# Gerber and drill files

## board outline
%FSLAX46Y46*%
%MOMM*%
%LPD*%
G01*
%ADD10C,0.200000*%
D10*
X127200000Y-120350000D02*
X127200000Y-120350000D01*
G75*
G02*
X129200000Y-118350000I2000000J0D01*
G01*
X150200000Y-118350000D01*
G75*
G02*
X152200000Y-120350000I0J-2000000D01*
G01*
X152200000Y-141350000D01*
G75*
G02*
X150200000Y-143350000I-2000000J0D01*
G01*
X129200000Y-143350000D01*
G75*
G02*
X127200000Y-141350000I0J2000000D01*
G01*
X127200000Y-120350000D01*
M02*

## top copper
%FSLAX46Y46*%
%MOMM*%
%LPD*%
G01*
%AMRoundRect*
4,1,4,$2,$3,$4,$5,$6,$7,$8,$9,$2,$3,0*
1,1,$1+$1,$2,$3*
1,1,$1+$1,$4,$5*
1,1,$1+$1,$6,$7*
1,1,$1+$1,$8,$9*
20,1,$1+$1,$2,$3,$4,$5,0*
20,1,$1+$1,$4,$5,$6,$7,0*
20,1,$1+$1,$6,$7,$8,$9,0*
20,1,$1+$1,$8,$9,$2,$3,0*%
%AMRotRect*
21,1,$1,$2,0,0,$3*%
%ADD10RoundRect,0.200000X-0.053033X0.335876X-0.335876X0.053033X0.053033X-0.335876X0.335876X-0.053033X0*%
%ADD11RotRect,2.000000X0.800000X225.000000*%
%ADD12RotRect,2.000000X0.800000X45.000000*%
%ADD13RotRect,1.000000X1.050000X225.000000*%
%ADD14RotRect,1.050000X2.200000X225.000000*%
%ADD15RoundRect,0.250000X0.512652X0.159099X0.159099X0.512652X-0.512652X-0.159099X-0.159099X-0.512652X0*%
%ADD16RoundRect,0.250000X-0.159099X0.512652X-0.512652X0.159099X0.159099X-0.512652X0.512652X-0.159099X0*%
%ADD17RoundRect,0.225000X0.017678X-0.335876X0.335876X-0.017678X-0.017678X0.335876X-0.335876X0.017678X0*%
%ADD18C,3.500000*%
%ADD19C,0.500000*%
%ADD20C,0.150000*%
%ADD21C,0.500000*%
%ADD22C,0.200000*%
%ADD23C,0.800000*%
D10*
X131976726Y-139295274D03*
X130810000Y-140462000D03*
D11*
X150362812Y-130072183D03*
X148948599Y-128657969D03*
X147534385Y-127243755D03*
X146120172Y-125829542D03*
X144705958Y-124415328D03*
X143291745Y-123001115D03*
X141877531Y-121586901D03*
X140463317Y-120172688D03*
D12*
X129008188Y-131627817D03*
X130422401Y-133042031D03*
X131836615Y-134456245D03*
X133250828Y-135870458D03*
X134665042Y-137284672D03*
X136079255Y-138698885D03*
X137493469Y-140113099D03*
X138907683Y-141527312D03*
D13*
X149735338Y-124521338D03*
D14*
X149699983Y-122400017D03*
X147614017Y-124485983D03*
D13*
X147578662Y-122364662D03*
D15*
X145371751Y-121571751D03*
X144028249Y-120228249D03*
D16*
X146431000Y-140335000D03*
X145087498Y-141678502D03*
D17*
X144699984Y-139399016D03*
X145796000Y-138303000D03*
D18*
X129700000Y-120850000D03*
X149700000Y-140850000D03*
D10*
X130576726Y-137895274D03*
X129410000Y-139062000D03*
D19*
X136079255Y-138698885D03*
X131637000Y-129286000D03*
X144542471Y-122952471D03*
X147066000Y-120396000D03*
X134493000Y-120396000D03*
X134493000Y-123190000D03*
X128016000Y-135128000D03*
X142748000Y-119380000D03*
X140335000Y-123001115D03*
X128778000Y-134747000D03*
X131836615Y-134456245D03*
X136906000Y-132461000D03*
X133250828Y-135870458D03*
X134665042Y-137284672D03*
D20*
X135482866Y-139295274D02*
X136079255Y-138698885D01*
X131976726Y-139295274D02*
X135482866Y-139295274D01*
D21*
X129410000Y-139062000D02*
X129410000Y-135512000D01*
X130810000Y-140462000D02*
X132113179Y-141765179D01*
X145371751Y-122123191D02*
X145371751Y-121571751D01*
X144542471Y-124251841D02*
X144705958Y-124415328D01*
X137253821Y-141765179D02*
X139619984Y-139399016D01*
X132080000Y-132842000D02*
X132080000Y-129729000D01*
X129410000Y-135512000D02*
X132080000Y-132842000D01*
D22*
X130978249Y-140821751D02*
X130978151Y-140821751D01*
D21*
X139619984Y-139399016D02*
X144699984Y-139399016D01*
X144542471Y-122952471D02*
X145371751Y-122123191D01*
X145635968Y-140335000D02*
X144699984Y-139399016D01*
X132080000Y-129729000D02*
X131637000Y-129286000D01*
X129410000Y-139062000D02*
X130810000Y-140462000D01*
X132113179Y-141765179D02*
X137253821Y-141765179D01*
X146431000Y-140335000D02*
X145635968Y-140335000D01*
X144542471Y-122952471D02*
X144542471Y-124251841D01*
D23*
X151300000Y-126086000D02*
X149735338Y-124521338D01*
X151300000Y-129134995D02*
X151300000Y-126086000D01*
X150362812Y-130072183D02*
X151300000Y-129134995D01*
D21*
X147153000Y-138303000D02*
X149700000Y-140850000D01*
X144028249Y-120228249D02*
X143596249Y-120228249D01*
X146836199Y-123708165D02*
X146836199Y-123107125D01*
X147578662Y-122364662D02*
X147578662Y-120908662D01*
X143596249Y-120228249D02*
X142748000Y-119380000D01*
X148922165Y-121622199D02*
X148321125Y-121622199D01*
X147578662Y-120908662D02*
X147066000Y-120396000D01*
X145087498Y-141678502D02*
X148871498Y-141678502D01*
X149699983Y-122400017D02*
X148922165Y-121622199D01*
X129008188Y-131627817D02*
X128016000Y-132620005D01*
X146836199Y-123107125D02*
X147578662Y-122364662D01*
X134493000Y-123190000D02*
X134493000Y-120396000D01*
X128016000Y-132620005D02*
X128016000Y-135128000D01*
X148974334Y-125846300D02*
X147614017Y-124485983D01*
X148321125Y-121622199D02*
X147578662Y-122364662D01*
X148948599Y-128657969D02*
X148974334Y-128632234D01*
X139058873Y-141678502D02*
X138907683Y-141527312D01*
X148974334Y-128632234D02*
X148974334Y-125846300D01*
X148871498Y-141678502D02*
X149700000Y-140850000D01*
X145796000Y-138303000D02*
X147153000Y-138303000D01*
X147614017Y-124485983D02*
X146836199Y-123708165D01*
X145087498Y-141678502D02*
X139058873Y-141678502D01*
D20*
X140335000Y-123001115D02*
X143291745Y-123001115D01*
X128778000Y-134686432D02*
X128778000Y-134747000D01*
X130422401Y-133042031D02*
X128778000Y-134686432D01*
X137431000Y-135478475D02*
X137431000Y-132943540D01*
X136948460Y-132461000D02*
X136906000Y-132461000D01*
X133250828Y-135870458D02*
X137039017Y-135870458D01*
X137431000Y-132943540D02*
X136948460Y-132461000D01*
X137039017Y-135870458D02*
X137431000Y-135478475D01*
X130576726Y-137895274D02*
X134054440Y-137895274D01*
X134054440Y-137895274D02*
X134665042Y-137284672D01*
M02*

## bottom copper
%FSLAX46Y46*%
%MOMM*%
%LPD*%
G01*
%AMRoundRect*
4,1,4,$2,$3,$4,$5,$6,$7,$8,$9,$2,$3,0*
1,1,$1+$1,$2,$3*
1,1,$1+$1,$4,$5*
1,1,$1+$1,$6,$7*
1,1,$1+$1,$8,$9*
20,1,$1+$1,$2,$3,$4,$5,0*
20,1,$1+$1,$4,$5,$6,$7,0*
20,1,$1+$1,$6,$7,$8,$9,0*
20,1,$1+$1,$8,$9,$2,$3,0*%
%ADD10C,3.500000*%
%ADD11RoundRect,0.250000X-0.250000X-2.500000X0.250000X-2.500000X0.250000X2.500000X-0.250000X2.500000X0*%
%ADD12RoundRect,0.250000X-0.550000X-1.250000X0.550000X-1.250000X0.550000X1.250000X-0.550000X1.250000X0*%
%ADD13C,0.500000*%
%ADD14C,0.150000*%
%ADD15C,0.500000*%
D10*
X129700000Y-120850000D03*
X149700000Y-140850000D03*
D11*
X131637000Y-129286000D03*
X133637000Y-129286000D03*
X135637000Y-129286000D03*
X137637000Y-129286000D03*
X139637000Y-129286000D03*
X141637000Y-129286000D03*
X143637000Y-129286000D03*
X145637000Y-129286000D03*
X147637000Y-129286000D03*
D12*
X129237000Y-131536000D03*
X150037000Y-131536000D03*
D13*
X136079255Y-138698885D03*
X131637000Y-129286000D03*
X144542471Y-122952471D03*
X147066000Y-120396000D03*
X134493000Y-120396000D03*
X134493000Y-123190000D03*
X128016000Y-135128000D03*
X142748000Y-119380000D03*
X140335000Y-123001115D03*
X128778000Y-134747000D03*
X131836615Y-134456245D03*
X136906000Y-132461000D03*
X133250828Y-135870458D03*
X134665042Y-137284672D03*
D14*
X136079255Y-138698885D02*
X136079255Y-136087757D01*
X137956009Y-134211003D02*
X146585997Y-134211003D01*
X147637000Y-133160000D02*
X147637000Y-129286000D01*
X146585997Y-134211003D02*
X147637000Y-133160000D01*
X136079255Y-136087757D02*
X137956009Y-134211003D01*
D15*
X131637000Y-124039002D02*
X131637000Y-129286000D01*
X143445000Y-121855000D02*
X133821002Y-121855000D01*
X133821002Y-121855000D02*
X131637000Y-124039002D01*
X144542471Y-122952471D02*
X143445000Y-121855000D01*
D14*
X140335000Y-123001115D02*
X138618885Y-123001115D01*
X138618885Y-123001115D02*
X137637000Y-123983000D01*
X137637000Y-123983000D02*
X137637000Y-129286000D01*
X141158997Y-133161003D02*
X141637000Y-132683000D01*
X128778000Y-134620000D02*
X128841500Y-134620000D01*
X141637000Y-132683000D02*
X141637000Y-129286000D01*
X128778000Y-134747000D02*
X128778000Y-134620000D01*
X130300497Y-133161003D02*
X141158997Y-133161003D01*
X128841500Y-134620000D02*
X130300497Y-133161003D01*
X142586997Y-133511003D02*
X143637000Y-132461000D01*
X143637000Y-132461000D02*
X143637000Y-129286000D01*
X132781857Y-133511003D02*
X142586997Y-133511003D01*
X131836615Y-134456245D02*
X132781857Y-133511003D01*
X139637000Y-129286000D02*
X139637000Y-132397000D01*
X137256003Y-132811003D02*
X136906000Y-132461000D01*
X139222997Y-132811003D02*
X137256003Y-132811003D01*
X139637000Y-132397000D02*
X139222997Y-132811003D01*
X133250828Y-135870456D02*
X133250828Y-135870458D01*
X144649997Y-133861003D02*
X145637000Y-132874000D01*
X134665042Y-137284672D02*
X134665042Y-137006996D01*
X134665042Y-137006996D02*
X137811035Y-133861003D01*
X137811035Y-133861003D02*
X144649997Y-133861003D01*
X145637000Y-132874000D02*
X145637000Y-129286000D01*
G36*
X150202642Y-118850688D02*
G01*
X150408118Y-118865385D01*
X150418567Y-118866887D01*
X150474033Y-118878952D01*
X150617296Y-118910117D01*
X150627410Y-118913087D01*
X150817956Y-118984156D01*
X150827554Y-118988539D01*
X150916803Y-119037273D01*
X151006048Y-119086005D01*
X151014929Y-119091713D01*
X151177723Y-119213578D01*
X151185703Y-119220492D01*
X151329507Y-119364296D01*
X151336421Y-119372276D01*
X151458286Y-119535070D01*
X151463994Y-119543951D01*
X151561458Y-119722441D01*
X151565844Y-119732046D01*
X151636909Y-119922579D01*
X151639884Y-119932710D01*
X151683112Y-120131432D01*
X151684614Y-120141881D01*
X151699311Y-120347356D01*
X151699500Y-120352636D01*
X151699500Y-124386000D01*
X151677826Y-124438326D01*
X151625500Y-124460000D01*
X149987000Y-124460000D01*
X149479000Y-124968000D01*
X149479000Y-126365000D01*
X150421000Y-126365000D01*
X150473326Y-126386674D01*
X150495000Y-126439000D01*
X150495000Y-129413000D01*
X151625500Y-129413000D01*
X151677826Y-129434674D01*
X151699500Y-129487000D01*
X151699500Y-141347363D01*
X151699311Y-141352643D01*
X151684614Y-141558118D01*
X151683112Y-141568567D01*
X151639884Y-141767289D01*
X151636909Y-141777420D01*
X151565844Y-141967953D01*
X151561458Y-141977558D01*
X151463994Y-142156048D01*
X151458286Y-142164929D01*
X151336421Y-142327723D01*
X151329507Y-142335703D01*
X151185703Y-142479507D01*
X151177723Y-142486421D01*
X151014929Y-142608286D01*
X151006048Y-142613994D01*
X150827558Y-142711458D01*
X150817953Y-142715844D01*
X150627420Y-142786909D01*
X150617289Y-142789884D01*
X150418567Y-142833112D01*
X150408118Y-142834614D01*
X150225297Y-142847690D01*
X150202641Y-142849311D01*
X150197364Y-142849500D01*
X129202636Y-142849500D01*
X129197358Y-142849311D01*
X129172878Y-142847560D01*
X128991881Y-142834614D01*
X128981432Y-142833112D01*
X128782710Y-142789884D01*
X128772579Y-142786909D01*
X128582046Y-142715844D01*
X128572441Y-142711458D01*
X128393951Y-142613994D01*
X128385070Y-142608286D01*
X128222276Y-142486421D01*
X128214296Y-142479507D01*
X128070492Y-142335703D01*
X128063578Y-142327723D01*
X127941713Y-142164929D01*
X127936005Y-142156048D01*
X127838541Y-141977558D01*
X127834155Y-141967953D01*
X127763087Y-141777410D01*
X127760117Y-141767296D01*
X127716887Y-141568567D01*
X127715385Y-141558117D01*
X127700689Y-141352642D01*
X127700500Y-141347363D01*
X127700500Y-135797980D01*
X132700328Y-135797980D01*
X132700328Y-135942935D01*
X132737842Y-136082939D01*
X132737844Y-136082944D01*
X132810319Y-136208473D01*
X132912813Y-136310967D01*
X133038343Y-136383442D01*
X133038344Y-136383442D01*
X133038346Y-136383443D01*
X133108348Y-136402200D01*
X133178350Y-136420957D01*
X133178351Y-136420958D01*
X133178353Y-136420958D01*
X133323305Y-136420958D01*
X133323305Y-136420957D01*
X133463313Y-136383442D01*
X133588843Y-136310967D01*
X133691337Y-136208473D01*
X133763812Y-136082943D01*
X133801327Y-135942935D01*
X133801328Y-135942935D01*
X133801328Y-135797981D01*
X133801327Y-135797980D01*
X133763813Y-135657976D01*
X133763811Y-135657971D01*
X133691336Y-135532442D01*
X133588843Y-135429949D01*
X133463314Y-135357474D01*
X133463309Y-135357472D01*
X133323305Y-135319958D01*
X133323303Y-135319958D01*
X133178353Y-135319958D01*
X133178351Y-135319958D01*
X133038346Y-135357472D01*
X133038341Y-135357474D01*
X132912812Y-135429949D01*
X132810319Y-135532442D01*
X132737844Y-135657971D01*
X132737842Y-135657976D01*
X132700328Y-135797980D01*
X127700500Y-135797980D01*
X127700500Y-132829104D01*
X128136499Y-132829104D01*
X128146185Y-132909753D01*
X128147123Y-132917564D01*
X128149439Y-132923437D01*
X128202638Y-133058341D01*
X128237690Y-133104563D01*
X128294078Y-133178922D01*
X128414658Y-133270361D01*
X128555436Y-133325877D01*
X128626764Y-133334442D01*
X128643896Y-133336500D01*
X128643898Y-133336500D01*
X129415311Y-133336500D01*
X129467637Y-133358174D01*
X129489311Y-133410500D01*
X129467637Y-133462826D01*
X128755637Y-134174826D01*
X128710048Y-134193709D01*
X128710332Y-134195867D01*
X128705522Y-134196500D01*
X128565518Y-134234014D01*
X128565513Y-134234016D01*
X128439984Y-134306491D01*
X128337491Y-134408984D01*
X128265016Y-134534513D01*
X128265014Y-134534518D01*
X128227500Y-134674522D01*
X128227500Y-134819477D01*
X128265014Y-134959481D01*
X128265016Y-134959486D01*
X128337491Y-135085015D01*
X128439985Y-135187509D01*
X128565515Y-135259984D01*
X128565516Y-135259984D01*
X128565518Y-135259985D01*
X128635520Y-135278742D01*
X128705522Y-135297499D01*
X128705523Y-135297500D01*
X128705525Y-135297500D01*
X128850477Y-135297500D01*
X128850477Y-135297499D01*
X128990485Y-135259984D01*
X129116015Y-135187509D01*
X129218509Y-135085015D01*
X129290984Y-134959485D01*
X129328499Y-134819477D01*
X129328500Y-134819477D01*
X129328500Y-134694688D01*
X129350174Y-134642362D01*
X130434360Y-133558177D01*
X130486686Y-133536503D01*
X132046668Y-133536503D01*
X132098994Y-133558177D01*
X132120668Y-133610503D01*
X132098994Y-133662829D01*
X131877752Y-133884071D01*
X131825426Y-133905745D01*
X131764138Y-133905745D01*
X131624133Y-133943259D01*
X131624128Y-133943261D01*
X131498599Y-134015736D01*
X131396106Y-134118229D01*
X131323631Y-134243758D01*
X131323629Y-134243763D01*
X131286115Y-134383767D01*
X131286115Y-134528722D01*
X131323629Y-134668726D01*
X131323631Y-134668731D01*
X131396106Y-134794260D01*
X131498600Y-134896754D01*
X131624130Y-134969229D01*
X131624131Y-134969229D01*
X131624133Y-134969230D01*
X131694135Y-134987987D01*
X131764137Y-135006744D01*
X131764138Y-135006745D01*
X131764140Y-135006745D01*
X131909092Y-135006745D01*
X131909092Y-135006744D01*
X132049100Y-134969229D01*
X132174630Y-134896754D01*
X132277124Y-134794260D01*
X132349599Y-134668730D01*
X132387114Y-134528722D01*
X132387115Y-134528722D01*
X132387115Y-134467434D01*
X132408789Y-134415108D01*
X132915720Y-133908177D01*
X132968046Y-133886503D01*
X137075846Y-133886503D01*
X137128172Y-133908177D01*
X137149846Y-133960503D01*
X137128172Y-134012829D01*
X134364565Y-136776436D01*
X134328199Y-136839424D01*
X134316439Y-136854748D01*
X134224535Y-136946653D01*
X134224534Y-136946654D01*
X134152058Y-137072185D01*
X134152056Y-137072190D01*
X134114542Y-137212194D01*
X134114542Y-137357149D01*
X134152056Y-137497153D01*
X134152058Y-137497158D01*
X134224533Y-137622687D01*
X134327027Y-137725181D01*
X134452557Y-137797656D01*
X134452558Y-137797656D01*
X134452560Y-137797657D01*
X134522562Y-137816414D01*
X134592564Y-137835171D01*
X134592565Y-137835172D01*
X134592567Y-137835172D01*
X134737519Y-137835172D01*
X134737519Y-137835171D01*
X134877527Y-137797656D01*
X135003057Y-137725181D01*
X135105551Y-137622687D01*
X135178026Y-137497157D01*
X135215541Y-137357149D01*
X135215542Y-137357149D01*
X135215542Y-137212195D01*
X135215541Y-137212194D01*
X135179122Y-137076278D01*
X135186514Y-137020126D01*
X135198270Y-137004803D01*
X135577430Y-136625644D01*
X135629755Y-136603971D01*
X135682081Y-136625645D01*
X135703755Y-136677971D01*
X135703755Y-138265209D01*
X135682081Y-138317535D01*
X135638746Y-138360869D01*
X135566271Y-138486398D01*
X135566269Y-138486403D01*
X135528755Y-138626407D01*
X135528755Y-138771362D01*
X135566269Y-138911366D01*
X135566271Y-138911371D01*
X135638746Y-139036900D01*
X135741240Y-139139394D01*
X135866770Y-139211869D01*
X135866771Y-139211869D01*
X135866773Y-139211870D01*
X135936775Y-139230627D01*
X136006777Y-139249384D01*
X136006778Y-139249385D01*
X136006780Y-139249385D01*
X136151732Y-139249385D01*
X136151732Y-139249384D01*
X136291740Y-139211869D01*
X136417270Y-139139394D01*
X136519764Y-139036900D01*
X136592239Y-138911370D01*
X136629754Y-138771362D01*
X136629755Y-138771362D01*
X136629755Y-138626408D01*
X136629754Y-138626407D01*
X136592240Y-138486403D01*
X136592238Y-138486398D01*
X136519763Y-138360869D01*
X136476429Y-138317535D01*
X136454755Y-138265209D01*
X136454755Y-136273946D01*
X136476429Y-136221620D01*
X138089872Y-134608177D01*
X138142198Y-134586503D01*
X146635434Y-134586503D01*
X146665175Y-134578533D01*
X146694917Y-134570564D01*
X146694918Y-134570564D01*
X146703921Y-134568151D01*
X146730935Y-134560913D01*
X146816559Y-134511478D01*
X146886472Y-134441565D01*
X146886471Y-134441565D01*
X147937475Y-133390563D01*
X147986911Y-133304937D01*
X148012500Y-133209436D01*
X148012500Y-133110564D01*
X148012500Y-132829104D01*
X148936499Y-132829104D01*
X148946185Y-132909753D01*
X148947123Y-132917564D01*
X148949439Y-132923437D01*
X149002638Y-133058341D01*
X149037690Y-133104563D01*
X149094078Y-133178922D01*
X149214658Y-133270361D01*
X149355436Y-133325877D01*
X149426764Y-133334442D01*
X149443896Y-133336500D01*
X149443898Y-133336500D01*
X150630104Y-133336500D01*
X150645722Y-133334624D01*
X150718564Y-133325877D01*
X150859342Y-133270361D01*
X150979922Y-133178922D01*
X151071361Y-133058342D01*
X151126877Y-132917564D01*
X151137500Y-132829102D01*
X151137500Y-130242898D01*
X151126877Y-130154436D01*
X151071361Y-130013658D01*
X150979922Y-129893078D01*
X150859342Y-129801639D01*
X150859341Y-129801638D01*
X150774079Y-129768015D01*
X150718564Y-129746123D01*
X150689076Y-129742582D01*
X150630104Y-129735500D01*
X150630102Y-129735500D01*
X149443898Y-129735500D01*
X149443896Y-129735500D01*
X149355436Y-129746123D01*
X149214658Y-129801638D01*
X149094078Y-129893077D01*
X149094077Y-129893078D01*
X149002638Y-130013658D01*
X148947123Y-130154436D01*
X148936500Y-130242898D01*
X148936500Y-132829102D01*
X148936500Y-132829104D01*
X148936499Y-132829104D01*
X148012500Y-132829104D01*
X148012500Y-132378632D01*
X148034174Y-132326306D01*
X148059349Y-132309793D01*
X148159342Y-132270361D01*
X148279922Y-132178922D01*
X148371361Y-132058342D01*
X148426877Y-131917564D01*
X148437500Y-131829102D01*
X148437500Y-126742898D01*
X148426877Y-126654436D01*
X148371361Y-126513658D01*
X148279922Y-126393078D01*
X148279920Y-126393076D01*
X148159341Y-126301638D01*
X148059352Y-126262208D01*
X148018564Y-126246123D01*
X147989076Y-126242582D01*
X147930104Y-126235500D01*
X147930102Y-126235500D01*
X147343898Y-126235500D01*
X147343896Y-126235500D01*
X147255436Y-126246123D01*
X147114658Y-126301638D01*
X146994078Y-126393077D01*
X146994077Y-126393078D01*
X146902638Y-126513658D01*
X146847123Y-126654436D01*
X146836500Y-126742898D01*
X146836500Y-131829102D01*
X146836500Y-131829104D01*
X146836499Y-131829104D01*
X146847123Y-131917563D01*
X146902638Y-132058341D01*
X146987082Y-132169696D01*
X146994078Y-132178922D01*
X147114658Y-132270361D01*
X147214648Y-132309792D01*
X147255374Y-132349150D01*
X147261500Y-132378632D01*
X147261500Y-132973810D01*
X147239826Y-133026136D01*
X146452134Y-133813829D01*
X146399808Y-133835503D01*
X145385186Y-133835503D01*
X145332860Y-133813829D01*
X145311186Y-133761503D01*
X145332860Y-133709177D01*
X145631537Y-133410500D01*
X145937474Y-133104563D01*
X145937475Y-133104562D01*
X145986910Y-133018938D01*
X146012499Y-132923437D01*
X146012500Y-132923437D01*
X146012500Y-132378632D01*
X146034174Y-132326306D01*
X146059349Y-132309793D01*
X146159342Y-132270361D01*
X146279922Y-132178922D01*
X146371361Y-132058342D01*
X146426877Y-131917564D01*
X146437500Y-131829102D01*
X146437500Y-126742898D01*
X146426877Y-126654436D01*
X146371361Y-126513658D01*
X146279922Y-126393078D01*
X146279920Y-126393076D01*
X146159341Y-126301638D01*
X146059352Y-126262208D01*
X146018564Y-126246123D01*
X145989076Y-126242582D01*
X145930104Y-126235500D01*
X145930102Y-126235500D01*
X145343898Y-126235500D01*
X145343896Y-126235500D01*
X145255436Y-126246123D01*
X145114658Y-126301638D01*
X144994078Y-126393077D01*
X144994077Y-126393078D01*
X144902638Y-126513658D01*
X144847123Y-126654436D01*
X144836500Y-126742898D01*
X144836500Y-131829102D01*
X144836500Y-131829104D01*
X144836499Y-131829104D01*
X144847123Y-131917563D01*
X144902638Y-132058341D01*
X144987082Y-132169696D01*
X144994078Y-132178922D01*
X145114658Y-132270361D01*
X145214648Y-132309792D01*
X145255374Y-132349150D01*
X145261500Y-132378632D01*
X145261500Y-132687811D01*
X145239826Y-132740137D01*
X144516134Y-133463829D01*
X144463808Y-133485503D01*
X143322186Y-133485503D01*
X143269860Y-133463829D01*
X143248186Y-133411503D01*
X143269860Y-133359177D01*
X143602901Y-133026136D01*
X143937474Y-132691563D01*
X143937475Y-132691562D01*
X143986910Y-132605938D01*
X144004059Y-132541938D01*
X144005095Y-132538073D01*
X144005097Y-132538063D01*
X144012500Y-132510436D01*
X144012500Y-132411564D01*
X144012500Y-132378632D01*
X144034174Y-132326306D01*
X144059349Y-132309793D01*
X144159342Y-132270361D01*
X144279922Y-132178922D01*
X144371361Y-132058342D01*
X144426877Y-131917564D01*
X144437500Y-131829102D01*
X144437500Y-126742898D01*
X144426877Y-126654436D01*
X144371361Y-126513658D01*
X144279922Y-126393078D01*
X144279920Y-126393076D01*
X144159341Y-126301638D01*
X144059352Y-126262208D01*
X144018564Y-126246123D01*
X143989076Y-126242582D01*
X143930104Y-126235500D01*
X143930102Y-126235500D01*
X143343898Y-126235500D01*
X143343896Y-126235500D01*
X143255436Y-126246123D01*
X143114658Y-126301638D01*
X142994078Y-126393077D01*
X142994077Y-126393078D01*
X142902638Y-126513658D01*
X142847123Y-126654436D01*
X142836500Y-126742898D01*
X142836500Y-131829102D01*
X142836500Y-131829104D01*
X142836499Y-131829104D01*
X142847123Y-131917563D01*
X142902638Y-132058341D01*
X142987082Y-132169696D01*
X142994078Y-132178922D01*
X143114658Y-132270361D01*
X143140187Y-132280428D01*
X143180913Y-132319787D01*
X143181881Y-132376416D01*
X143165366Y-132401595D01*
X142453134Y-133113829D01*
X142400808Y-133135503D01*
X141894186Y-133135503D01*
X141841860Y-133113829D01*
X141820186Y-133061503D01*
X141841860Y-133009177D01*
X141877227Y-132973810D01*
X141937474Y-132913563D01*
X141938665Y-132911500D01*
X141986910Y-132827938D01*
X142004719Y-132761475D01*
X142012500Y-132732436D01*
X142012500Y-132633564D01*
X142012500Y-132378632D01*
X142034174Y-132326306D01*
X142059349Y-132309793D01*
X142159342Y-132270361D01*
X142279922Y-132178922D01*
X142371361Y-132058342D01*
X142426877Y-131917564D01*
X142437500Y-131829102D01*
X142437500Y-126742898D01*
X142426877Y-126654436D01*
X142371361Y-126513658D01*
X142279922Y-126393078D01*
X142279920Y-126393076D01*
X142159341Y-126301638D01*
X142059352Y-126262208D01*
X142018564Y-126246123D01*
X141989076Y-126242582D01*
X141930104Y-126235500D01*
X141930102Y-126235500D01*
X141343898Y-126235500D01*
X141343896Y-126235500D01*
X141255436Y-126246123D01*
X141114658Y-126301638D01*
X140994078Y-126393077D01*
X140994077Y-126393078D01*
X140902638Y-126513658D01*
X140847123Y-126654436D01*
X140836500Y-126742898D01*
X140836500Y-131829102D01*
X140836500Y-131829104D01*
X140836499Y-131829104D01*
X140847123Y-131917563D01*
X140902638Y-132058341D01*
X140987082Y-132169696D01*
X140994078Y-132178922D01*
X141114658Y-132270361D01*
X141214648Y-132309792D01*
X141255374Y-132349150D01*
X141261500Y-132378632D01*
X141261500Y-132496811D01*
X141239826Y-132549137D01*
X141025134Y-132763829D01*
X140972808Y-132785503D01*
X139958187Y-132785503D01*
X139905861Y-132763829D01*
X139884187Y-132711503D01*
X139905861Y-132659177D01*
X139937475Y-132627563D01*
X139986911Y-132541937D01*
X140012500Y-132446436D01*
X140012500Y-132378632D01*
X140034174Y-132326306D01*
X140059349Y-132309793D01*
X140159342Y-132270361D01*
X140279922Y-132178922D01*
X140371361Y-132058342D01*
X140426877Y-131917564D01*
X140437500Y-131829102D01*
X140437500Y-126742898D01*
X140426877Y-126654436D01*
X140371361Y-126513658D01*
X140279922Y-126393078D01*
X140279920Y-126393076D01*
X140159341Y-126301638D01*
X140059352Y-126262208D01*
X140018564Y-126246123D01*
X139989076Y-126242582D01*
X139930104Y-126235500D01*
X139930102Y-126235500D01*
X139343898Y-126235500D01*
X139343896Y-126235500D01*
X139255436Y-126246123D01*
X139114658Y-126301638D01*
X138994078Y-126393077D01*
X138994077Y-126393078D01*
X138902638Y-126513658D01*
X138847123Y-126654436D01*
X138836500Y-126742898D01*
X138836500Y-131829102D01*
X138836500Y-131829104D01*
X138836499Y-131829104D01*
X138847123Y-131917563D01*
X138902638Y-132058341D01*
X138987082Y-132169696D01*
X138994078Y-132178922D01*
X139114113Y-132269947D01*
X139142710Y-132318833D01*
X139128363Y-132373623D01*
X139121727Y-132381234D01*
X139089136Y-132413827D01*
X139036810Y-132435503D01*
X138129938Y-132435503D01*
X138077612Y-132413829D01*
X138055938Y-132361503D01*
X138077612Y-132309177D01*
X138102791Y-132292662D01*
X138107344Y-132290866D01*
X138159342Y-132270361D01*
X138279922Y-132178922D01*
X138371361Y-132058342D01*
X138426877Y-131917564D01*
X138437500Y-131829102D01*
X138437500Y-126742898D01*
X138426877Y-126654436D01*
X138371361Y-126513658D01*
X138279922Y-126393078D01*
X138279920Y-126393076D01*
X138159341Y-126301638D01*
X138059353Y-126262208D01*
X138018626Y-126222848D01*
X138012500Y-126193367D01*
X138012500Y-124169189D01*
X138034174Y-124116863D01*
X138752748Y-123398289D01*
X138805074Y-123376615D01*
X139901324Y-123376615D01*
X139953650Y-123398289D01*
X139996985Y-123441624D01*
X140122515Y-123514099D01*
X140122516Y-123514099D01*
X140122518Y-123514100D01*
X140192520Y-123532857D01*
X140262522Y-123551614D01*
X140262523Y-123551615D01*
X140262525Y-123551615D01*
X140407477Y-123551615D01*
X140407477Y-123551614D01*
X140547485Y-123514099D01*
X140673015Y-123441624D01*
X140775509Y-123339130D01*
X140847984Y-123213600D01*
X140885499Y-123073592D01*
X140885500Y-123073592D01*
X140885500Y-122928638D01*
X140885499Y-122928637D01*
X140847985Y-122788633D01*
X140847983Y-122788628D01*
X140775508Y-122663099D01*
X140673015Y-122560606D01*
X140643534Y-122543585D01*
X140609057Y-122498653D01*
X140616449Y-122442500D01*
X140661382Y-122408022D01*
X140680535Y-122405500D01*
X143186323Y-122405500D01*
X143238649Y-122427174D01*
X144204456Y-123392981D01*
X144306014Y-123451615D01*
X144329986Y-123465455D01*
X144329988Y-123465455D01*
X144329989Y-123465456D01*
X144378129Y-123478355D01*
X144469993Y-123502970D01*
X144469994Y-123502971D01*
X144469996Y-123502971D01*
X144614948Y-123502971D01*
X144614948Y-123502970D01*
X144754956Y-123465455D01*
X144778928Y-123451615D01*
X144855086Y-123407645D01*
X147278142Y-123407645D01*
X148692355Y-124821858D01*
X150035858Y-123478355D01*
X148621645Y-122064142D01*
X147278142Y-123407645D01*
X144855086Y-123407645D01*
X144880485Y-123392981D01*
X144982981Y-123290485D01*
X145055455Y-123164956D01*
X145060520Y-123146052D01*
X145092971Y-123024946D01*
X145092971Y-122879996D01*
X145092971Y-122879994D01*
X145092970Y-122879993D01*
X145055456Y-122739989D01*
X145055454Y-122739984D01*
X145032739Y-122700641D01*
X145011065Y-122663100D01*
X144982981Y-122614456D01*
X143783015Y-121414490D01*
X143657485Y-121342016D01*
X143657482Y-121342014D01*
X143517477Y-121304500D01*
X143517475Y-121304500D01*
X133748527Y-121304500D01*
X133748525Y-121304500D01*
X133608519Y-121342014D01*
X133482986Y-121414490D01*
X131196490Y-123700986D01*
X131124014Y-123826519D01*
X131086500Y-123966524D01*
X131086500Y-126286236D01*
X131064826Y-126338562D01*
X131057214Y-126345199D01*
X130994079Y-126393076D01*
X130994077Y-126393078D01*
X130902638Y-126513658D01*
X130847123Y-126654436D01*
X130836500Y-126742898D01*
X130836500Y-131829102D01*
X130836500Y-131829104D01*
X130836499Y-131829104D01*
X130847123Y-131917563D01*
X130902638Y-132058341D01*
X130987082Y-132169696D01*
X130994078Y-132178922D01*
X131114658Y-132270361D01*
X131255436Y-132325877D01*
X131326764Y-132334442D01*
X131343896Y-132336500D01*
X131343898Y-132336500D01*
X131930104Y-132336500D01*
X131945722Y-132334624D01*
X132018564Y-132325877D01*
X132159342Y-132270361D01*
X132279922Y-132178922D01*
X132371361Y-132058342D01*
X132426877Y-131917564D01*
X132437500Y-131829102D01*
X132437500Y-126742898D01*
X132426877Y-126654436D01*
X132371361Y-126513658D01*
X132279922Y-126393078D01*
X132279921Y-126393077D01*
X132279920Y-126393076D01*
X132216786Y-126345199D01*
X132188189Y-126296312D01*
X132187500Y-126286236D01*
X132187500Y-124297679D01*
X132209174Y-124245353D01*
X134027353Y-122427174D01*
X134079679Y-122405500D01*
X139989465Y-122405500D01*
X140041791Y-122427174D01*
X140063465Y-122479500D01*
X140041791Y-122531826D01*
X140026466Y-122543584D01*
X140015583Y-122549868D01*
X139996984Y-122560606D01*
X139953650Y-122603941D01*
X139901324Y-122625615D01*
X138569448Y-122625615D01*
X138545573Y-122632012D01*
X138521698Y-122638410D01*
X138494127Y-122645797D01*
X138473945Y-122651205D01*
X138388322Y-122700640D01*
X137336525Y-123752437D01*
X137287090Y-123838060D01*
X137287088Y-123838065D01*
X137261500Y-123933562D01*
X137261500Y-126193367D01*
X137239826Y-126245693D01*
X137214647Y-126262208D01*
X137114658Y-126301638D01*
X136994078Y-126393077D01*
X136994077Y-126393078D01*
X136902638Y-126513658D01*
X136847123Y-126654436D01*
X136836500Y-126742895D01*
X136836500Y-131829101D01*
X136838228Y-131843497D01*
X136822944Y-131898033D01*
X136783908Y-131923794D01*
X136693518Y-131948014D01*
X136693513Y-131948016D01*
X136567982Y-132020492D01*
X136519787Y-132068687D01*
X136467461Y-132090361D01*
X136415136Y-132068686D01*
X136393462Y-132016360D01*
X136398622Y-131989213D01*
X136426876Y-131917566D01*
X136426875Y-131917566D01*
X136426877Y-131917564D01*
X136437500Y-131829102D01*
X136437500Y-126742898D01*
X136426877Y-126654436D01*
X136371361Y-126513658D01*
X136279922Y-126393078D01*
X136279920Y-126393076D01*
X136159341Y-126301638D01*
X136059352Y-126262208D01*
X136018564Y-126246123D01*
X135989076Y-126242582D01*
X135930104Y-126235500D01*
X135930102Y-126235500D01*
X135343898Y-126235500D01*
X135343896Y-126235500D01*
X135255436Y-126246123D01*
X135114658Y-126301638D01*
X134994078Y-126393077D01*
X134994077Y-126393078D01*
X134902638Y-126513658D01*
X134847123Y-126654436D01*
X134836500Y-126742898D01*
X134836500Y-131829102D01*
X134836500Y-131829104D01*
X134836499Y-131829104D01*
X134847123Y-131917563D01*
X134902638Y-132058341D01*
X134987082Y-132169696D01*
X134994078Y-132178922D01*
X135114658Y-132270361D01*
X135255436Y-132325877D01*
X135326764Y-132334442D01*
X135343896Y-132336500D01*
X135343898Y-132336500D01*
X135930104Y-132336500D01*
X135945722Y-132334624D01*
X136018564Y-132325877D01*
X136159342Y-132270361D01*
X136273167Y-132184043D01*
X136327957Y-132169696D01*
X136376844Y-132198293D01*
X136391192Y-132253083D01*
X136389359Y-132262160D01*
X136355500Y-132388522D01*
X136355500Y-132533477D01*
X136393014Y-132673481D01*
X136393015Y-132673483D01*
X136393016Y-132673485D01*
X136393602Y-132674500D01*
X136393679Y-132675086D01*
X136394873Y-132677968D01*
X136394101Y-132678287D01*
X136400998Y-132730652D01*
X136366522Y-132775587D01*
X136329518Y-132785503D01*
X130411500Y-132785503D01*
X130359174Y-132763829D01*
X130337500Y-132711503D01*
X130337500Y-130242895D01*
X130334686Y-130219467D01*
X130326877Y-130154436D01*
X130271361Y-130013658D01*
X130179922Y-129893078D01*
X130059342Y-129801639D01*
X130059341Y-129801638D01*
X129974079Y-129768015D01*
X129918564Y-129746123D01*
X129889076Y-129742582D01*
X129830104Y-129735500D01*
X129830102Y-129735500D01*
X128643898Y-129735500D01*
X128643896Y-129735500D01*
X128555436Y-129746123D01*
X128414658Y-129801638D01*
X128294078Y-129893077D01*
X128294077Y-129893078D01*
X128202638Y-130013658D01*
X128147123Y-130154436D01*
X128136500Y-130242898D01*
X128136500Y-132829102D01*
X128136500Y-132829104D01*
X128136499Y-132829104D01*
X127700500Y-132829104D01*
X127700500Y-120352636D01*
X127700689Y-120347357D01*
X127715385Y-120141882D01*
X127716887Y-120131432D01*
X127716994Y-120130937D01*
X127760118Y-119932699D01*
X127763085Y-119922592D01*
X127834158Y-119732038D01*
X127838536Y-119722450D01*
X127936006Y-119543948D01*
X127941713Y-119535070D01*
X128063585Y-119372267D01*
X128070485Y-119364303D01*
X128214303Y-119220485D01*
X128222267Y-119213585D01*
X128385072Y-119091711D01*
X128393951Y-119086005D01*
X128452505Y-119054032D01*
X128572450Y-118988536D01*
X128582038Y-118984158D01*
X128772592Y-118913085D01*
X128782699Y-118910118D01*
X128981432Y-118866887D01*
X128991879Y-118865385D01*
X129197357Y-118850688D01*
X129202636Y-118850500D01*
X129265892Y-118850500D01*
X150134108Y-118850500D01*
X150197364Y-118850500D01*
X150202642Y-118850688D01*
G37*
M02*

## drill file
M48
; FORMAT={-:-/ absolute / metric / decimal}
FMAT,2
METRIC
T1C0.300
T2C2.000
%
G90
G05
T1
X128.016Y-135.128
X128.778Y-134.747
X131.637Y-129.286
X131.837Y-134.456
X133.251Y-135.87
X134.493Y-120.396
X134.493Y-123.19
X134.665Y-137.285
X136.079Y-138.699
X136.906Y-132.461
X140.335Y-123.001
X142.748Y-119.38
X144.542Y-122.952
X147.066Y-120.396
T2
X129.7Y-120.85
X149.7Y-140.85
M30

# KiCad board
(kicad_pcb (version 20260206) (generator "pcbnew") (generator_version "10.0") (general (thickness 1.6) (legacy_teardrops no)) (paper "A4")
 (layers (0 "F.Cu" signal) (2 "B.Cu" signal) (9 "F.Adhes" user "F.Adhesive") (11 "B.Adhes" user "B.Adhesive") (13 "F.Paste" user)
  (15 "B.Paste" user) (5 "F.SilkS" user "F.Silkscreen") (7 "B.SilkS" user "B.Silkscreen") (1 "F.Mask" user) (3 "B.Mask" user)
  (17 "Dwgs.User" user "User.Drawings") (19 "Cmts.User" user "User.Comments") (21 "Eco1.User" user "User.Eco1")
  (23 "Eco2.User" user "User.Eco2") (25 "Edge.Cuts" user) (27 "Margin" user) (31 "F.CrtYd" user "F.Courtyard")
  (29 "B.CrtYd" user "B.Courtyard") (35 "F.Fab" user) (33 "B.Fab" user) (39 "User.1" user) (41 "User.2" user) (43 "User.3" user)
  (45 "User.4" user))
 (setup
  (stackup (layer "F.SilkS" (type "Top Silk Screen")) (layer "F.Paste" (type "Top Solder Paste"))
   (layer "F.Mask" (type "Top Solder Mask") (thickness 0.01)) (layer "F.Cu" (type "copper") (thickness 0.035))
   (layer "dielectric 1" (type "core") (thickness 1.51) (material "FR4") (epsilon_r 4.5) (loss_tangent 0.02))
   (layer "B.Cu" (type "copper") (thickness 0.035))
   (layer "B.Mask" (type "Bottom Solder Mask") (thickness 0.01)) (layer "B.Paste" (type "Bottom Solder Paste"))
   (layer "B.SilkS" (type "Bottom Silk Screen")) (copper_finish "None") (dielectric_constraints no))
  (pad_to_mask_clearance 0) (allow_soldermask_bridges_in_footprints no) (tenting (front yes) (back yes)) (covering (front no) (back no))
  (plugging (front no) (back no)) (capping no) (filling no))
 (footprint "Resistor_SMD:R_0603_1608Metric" (layer "F.Cu") (at 131.393363 139.878637 -135)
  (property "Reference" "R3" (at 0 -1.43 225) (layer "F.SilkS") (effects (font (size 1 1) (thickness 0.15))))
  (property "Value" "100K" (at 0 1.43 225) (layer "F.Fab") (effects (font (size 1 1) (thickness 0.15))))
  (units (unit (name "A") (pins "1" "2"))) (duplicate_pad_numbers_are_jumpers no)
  (pad "1" smd roundrect (at -0.825 0 225) (size 0.8 0.95) (layers "F.Cu" "F.Mask" "F.Paste") (roundrect_rratio 0.25) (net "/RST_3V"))
  (pad "2" smd roundrect (at 0.825 0 225) (size 0.8 0.95) (layers "F.Cu" "F.Mask" "F.Paste") (roundrect_rratio 0.25) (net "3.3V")))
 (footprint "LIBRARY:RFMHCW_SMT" (layer "F.Cu") (at 139.6855 130.85 45)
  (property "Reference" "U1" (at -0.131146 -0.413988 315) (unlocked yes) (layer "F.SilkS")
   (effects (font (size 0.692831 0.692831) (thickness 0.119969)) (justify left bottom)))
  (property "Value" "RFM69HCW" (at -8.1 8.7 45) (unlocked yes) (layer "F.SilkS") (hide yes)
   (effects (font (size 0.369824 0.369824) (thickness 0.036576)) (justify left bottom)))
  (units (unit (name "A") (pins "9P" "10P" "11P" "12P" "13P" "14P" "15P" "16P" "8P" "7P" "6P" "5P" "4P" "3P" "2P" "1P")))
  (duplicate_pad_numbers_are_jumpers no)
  (pad "1P" smd rect (at 8.099999 7 225) (size 2 0.8) (layers "F.Cu" "F.Mask" "F.Paste") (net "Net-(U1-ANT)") (solder_mask_margin 0.0508)
   (solder_paste_margin 0) (thermal_bridge_angle 0))
  (pad "2P" smd rect (at 8.1 5 225) (size 2 0.8) (layers "F.Cu" "F.Mask" "F.Paste") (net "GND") (solder_mask_margin 0.0508)
   (solder_paste_margin 0) (thermal_bridge_angle 0))
  (pad "3P" smd rect (at 8.1 3 225) (size 2 0.8) (layers "F.Cu" "F.Mask" "F.Paste") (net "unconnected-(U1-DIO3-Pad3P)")
   (solder_mask_margin 0.0508) (solder_paste_margin 0) (thermal_bridge_angle 0))
  (pad "4P" smd rect (at 8.1 1 225) (size 2 0.8) (layers "F.Cu" "F.Mask" "F.Paste") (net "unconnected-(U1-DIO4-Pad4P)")
   (solder_mask_margin 0.0508) (solder_paste_margin 0) (thermal_bridge_angle 0))
  (pad "5P" smd rect (at 8.1 -1 225) (size 2 0.8) (layers "F.Cu" "F.Mask" "F.Paste") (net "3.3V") (solder_mask_margin 0.0508)
   (solder_paste_margin 0) (thermal_bridge_angle 0))
  (pad "6P" smd rect (at 8.1 -3 225) (size 2 0.8) (layers "F.Cu" "F.Mask" "F.Paste") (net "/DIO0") (solder_mask_margin 0.0508)
   (solder_paste_margin 0) (thermal_bridge_angle 0))
  (pad "7P" smd rect (at 8.1 -5 225) (size 2 0.8) (layers "F.Cu" "F.Mask" "F.Paste") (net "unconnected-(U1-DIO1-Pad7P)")
   (solder_mask_margin 0.0508) (solder_paste_margin 0) (thermal_bridge_angle 0))
  (pad "8P" smd rect (at 8.099999 -7 225) (size 2 0.8) (layers "F.Cu" "F.Mask" "F.Paste") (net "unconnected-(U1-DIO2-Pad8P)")
   (solder_mask_margin 0.0508) (solder_paste_margin 0) (thermal_bridge_angle 0))
  (pad "9P" smd rect (at -8.099999 -7 45) (size 2 0.8) (layers "F.Cu" "F.Mask" "F.Paste") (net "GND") (solder_mask_margin 0.0508)
   (solder_paste_margin 0) (thermal_bridge_angle 0))
  (pad "10P" smd rect (at -8.1 -5 45) (size 2 0.8) (layers "F.Cu" "F.Mask" "F.Paste") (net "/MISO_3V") (solder_mask_margin 0.0508)
   (solder_paste_margin 0) (thermal_bridge_angle 0))
  (pad "11P" smd rect (at -8.1 -3 45) (size 2 0.8) (layers "F.Cu" "F.Mask" "F.Paste") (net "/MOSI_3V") (solder_mask_margin 0.0508)
   (solder_paste_margin 0) (thermal_bridge_angle 0))
  (pad "12P" smd rect (at -8.1 -1 45) (size 2 0.8) (layers "F.Cu" "F.Mask" "F.Paste") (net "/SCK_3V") (solder_mask_margin 0.0508)
   (solder_paste_margin 0) (thermal_bridge_angle 0))
  (pad "13P" smd rect (at -8.1 1 45) (size 2 0.8) (layers "F.Cu" "F.Mask" "F.Paste") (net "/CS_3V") (solder_mask_margin 0.0508)
   (solder_paste_margin 0) (thermal_bridge_angle 0))
  (pad "14P" smd rect (at -8.1 3 45) (size 2 0.8) (layers "F.Cu" "F.Mask" "F.Paste") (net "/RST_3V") (solder_mask_margin 0.0508)
   (solder_paste_margin 0) (thermal_bridge_angle 0))
  (pad "15P" smd rect (at -8.1 5 45) (size 2 0.8) (layers "F.Cu" "F.Mask" "F.Paste") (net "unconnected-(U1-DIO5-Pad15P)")
   (solder_mask_margin 0.0508) (solder_paste_margin 0) (thermal_bridge_angle 0))
  (pad "16P" smd rect (at -8.099999 7 45) (size 2 0.8) (layers "F.Cu" "F.Mask" "F.Paste") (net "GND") (solder_mask_margin 0.0508)
   (solder_paste_margin 0) (thermal_bridge_angle 0)))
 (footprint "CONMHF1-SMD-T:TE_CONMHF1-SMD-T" (layer "F.Cu") (at 148.657 123.443 -135)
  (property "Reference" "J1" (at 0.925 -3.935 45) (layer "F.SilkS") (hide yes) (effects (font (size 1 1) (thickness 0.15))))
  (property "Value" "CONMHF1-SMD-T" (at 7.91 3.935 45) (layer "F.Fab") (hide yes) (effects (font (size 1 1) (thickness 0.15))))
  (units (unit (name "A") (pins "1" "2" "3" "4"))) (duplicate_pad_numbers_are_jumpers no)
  (pad "1" smd rect (at 0 -1.525 225) (size 1 1.05) (layers "F.Cu" "F.Mask" "F.Paste") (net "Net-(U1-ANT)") (solder_mask_margin 0.102))
  (pad "2" smd rect (at -1.475001 0 225) (size 1.05 2.2) (layers "F.Cu" "F.Mask" "F.Paste") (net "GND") (solder_mask_margin 0.102))
  (pad "3" smd rect (at 1.475001 0 225) (size 1.05 2.2) (layers "F.Cu" "F.Mask" "F.Paste") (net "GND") (solder_mask_margin 0.102))
  (pad "4" smd rect (at 0 1.525 225) (size 1 1.05) (layers "F.Cu" "F.Mask" "F.Paste") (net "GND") (solder_mask_margin 0.102))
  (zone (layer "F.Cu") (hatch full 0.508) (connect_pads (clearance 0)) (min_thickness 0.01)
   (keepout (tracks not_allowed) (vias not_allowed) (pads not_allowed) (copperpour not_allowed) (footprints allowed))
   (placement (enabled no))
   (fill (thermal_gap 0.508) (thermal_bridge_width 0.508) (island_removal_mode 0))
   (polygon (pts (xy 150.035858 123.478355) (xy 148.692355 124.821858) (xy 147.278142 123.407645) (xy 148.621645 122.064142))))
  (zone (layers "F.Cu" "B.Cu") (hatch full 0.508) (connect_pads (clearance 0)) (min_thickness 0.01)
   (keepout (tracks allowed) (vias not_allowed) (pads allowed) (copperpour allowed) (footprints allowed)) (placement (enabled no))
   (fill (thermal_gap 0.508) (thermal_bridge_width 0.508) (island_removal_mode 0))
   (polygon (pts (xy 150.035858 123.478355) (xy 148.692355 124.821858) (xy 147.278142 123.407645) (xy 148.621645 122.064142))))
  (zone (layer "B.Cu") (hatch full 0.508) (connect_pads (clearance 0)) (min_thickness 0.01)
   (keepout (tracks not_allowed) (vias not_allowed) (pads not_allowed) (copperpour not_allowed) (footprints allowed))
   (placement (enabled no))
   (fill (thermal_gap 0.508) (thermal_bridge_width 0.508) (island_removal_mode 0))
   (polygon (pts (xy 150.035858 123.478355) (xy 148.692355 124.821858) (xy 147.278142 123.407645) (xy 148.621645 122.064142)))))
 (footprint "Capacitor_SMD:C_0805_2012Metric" (layer "F.Cu") (at 144.7 120.9 135)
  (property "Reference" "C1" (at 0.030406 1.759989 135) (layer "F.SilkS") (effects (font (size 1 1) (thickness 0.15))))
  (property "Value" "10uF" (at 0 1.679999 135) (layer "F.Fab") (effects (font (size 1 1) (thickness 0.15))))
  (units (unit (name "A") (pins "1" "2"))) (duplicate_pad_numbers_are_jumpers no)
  (pad "1" smd roundrect (at -0.949999 0 135) (size 1 1.45) (layers "F.Cu" "F.Mask" "F.Paste") (roundrect_rratio 0.25) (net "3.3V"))
  (pad "2" smd roundrect (at 0.949999 0 135) (size 1 1.45) (layers "F.Cu" "F.Mask" "F.Paste") (roundrect_rratio 0.25) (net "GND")))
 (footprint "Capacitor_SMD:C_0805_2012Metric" (layer "F.Cu") (at 145.759249 141.006751 -135)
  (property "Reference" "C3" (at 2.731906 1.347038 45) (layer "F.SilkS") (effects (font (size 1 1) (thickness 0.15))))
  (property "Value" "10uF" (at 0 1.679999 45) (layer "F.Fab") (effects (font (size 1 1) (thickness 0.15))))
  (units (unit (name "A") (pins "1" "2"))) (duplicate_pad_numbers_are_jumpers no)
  (pad "1" smd roundrect (at -0.949999 0 225) (size 1 1.45) (layers "F.Cu" "F.Mask" "F.Paste") (roundrect_rratio 0.25) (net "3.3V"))
  (pad "2" smd roundrect (at 0.949999 0 225) (size 1 1.45) (layers "F.Cu" "F.Mask" "F.Paste") (roundrect_rratio 0.25) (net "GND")))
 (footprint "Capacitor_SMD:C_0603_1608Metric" (layer "F.Cu") (at 145.247992 138.851008 45)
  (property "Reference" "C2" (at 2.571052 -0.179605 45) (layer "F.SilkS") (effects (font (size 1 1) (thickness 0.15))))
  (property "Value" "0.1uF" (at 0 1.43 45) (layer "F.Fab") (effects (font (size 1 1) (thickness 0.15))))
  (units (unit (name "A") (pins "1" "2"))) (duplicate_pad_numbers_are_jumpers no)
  (pad "1" smd roundrect (at -0.775 0 45) (size 0.9 0.95) (layers "F.Cu" "F.Mask" "F.Paste") (roundrect_rratio 0.25) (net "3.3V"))
  (pad "2" smd roundrect (at 0.775 0 45) (size 0.9 0.95) (layers "F.Cu" "F.Mask" "F.Paste") (roundrect_rratio 0.25) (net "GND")))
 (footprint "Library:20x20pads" (layer "F.Cu") (at 139.7 130.85)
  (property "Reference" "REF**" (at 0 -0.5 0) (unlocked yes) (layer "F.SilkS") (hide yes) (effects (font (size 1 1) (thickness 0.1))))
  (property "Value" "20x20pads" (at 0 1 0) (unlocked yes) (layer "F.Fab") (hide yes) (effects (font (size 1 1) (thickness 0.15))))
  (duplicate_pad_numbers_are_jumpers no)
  (pad "1" thru_hole circle (at -10 -10) (size 3.5 3.5) (drill 2) (layers "*.Cu" "*.Mask") (remove_unused_layers no) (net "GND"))
  (pad "1" thru_hole circle (at 10 10) (size 3.5 3.5) (drill 2) (layers "*.Cu" "*.Mask") (remove_unused_layers no) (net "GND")))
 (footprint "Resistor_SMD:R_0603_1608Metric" (layer "F.Cu") (at 129.993363 138.478637 -135)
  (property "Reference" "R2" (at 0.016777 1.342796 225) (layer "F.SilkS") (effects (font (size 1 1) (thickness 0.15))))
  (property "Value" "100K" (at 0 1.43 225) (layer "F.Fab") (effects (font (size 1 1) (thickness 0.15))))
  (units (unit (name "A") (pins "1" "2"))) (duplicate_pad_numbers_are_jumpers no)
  (pad "1" smd roundrect (at -0.825 0 225) (size 0.8 0.95) (layers "F.Cu" "F.Mask" "F.Paste") (roundrect_rratio 0.25) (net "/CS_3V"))
  (pad "2" smd roundrect (at 0.825 0 225) (size 0.8 0.95) (layers "F.Cu" "F.Mask" "F.Paste") (roundrect_rratio 0.25) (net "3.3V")))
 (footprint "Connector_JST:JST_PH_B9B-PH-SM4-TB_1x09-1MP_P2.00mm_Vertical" (layer "B.Cu") (at 139.637 129.786)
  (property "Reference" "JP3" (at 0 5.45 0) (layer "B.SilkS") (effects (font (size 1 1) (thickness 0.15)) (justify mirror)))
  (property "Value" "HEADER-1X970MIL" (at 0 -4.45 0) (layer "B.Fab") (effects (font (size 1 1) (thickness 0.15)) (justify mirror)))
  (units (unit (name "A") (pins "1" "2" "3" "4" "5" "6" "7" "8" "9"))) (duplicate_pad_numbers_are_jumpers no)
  (pad "1" smd roundrect (at -8 -0.5) (size 1 5.5) (layers "B.Cu" "B.Mask" "B.Paste") (roundrect_rratio 0.25) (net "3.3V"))
  (pad "2" smd roundrect (at -6 -0.5) (size 1 5.5) (layers "B.Cu" "B.Mask" "B.Paste") (roundrect_rratio 0.25) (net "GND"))
  (pad "3" smd roundrect (at -4 -0.5) (size 1 5.5) (layers "B.Cu" "B.Mask" "B.Paste") (roundrect_rratio 0.25) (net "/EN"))
  (pad "4" smd roundrect (at -2 -0.5) (size 1 5.5) (layers "B.Cu" "B.Mask" "B.Paste") (roundrect_rratio 0.25) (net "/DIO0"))
  (pad "5" smd roundrect (at 0 -0.5) (size 1 5.5) (layers "B.Cu" "B.Mask" "B.Paste") (roundrect_rratio 0.25) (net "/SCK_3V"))
  (pad "6" smd roundrect (at 2 -0.5) (size 1 5.5) (layers "B.Cu" "B.Mask" "B.Paste") (roundrect_rratio 0.25) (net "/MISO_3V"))
  (pad "7" smd roundrect (at 4 -0.5) (size 1 5.5) (layers "B.Cu" "B.Mask" "B.Paste") (roundrect_rratio 0.25) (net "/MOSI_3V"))
  (pad "8" smd roundrect (at 6 -0.5) (size 1 5.5) (layers "B.Cu" "B.Mask" "B.Paste") (roundrect_rratio 0.25) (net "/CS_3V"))
  (pad "9" smd roundrect (at 8 -0.5) (size 1 5.5) (layers "B.Cu" "B.Mask" "B.Paste") (roundrect_rratio 0.25) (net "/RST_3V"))
  (pad "MP" smd roundrect (at -10.4 1.75) (size 1.6 3) (layers "B.Cu" "B.Mask" "B.Paste") (roundrect_rratio 0.15625))
  (pad "MP" smd roundrect (at 10.4 1.75) (size 1.6 3) (layers "B.Cu" "B.Mask" "B.Paste") (roundrect_rratio 0.15625)))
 (gr_rect (start 127.2 118.35) (end 152.2 143.35) (radius 2) (stroke (width 0.2) (type solid)) (fill no) (layer "Edge.Cuts"))
 (segment (start 135.482866 139.295274) (end 136.079255 138.698885) (width 0.15) (layer "F.Cu") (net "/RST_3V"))
 (segment (start 131.976726 139.295274) (end 135.482866 139.295274) (width 0.15) (layer "F.Cu") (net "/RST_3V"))
 (via (at 136.079255 138.698885) (size 0.5) (drill 0.3) (layers "F.Cu" "B.Cu") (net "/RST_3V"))
 (segment (start 136.079255 138.698885) (end 136.079255 136.087757) (width 0.15) (layer "B.Cu") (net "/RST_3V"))
 (segment (start 137.956009 134.211003) (end 146.585997 134.211003) (width 0.15) (layer "B.Cu") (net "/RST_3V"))
 (segment (start 147.637 133.16) (end 147.637 129.286) (width 0.15) (layer "B.Cu") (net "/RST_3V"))
 (segment (start 146.585997 134.211003) (end 147.637 133.16) (width 0.15) (layer "B.Cu") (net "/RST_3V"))
 (segment (start 136.079255 136.087757) (end 137.956009 134.211003) (width 0.15) (layer "B.Cu") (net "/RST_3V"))
 (segment (start 129.41 139.062) (end 129.41 135.512) (width 0.5) (layer "F.Cu") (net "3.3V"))
 (segment (start 130.81 140.462) (end 132.113179 141.765179) (width 0.5) (layer "F.Cu") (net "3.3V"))
 (segment (start 145.371751 122.123191) (end 145.371751 121.571751) (width 0.5) (layer "F.Cu") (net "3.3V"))
 (segment (start 144.542471 124.251841) (end 144.705958 124.415328) (width 0.5) (layer "F.Cu") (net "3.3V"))
 (segment (start 137.253821 141.765179) (end 139.619984 139.399016) (width 0.5) (layer "F.Cu") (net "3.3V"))
 (segment (start 132.08 132.842) (end 132.08 129.729) (width 0.5) (layer "F.Cu") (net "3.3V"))
 (segment (start 129.41 135.512) (end 132.08 132.842) (width 0.5) (layer "F.Cu") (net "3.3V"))
 (segment (start 130.978249 140.821751) (end 130.978151 140.821751) (width 0.2) (layer "F.Cu") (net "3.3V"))
 (segment (start 139.619984 139.399016) (end 144.699984 139.399016) (width 0.5) (layer "F.Cu") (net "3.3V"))
 (segment (start 144.542471 122.952471) (end 145.371751 122.123191) (width 0.5) (layer "F.Cu") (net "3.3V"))
 (segment (start 145.635968 140.335) (end 144.699984 139.399016) (width 0.5) (layer "F.Cu") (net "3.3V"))
 (segment (start 132.08 129.729) (end 131.637 129.286) (width 0.5) (layer "F.Cu") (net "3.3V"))
 (segment (start 129.41 139.062) (end 130.81 140.462) (width 0.5) (layer "F.Cu") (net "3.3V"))
 (segment (start 132.113179 141.765179) (end 137.253821 141.765179) (width 0.5) (layer "F.Cu") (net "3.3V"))
 (segment (start 146.431 140.335) (end 145.635968 140.335) (width 0.5) (layer "F.Cu") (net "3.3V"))
 (segment (start 144.542471 122.952471) (end 144.542471 124.251841) (width 0.5) (layer "F.Cu") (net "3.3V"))
 (via (at 131.637 129.286) (size 0.5) (drill 0.3) (layers "F.Cu" "B.Cu") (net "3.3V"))
 (via (at 144.542471 122.952471) (size 0.5) (drill 0.3) (layers "F.Cu" "B.Cu") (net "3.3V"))
 (segment (start 131.637 124.039002) (end 131.637 129.286) (width 0.5) (layer "B.Cu") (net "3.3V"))
 (segment (start 143.445 121.855) (end 133.821002 121.855) (width 0.5) (layer "B.Cu") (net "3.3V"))
 (segment (start 133.821002 121.855) (end 131.637 124.039002) (width 0.5) (layer "B.Cu") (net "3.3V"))
 (segment (start 144.542471 122.952471) (end 143.445 121.855) (width 0.5) (layer "B.Cu") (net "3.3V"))
 (segment (start 151.3 126.086) (end 149.735338 124.521338) (width 0.8) (layer "F.Cu") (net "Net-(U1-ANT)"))
 (segment (start 151.3 129.134995) (end 151.3 126.086) (width 0.8) (layer "F.Cu") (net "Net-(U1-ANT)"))
 (segment (start 150.362812 130.072183) (end 151.3 129.134995) (width 0.8) (layer "F.Cu") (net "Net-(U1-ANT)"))
 (segment (start 147.153 138.303) (end 149.7 140.85) (width 0.5) (layer "F.Cu") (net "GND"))
 (segment (start 144.028249 120.228249) (end 143.596249 120.228249) (width 0.5) (layer "F.Cu") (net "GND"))
 (segment (start 146.836199 123.708165) (end 146.836199 123.107125) (width 0.5) (layer "F.Cu") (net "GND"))
 (segment (start 147.578662 122.364662) (end 147.578662 120.908662) (width 0.5) (layer "F.Cu") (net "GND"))
 (segment (start 143.596249 120.228249) (end 142.748 119.38) (width 0.5) (layer "F.Cu") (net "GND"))
 (segment (start 148.922165 121.622199) (end 148.321125 121.622199) (width 0.5) (layer "F.Cu") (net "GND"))
 (segment (start 147.578662 120.908662) (end 147.066 120.396) (width 0.5) (layer "F.Cu") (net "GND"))
 (segment (start 145.087498 141.678502) (end 148.871498 141.678502) (width 0.5) (layer "F.Cu") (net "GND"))
 (segment (start 149.699983 122.400017) (end 148.922165 121.622199) (width 0.5) (layer "F.Cu") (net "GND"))
 (segment (start 129.008188 131.627817) (end 128.016 132.620005) (width 0.5) (layer "F.Cu") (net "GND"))
 (segment (start 146.836199 123.107125) (end 147.578662 122.364662) (width 0.5) (layer "F.Cu") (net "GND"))
 (segment (start 134.493 123.19) (end 134.493 120.396) (width 0.5) (layer "F.Cu") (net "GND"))
 (segment (start 128.016 132.620005) (end 128.016 135.128) (width 0.5) (layer "F.Cu") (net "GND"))
 (segment (start 148.974334 125.8463) (end 147.614017 124.485983) (width 0.5) (layer "F.Cu") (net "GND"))
 (segment (start 148.321125 121.622199) (end 147.578662 122.364662) (width 0.5) (layer "F.Cu") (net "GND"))
 (segment (start 148.948599 128.657969) (end 148.974334 128.632234) (width 0.5) (layer "F.Cu") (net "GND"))
 (segment (start 139.058873 141.678502) (end 138.907683 141.527312) (width 0.5) (layer "F.Cu") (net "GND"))
 (segment (start 148.974334 128.632234) (end 148.974334 125.8463) (width 0.5) (layer "F.Cu") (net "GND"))
 (segment (start 148.871498 141.678502) (end 149.7 140.85) (width 0.5) (layer "F.Cu") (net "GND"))
 (segment (start 145.796 138.303) (end 147.153 138.303) (width 0.5) (layer "F.Cu") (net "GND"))
 (segment (start 147.614017 124.485983) (end 146.836199 123.708165) (width 0.5) (layer "F.Cu") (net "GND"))
 (segment (start 145.087498 141.678502) (end 139.058873 141.678502) (width 0.5) (layer "F.Cu") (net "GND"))
 (via (at 147.066 120.396) (size 0.5) (drill 0.3) (layers "F.Cu" "B.Cu") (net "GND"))
 (via (at 134.493 120.396) (size 0.5) (drill 0.3) (layers "F.Cu" "B.Cu") (free yes) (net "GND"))
 (via (at 134.493 123.19) (size 0.5) (drill 0.3) (layers "F.Cu" "B.Cu") (free yes) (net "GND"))
 (via (at 128.016 135.128) (size 0.5) (drill 0.3) (layers "F.Cu" "B.Cu") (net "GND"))
 (via (at 142.748 119.38) (size 0.5) (drill 0.3) (layers "F.Cu" "B.Cu") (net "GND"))
 (segment (start 140.335 123.001115) (end 143.291745 123.001115) (width 0.15) (layer "F.Cu") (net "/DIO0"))
 (via (at 140.335 123.001115) (size 0.5) (drill 0.3) (layers "F.Cu" "B.Cu") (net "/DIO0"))
 (segment (start 140.335 123.001115) (end 138.618885 123.001115) (width 0.15) (layer "B.Cu") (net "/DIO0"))
 (segment (start 138.618885 123.001115) (end 137.637 123.983) (width 0.15) (layer "B.Cu") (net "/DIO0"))
 (segment (start 137.637 123.983) (end 137.637 129.286) (width 0.15) (layer "B.Cu") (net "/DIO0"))
 (segment (start 128.778 134.686432) (end 128.778 134.747) (width 0.15) (layer "F.Cu") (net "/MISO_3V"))
 (segment (start 130.422401 133.042031) (end 128.778 134.686432) (width 0.15) (layer "F.Cu") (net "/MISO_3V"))
 (via (at 128.778 134.747) (size 0.5) (drill 0.3) (layers "F.Cu" "B.Cu") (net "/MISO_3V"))
 (segment (start 141.158997 133.161003) (end 141.637 132.683) (width 0.15) (layer "B.Cu") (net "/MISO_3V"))
 (segment (start 128.778 134.62) (end 128.8415 134.62) (width 0.15) (layer "B.Cu") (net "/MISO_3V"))
 (segment (start 141.637 132.683) (end 141.637 129.286) (width 0.15) (layer "B.Cu") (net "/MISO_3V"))
 (segment (start 128.778 134.747) (end 128.778 134.62) (width 0.15) (layer "B.Cu") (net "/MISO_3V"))
 (segment (start 130.300497 133.161003) (end 141.158997 133.161003) (width 0.15) (layer "B.Cu") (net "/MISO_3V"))
 (segment (start 128.8415 134.62) (end 130.300497 133.161003) (width 0.15) (layer "B.Cu") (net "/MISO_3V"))
 (via (at 131.836615 134.456245) (size 0.5) (drill 0.3) (layers "F.Cu" "B.Cu") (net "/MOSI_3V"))
 (segment (start 142.586997 133.511003) (end 143.637 132.461) (width 0.15) (layer "B.Cu") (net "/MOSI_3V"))
 (segment (start 143.637 132.461) (end 143.637 129.286) (width 0.15) (layer "B.Cu") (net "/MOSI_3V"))
 (segment (start 132.781857 133.511003) (end 142.586997 133.511003) (width 0.15) (layer "B.Cu") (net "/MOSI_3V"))
 (segment (start 131.836615 134.456245) (end 132.781857 133.511003) (width 0.15) (layer "B.Cu") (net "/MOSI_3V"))
 (segment (start 137.431 135.478475) (end 137.431 132.94354) (width 0.15) (layer "F.Cu") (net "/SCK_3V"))
 (segment (start 136.94846 132.461) (end 136.906 132.461) (width 0.15) (layer "F.Cu") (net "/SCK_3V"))
 (segment (start 133.250828 135.870458) (end 137.039017 135.870458) (width 0.15) (layer "F.Cu") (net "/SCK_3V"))
 (segment (start 137.431 132.94354) (end 136.94846 132.461) (width 0.15) (layer "F.Cu") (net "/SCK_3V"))
 (segment (start 137.039017 135.870458) (end 137.431 135.478475) (width 0.15) (layer "F.Cu") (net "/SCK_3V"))
 (via (at 136.906 132.461) (size 0.5) (drill 0.3) (layers "F.Cu" "B.Cu") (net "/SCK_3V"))
 (via (at 133.250828 135.870458) (size 0.5) (drill 0.3) (layers "F.Cu" "B.Cu") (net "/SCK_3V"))
 (segment (start 139.637 129.286) (end 139.637 132.397) (width 0.15) (layer "B.Cu") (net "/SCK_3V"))
 (segment (start 137.256003 132.811003) (end 136.906 132.461) (width 0.15) (layer "B.Cu") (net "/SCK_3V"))
 (segment (start 139.222997 132.811003) (end 137.256003 132.811003) (width 0.15) (layer "B.Cu") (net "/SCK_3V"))
 (segment (start 139.637 132.397) (end 139.222997 132.811003) (width 0.15) (layer "B.Cu") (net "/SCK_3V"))
 (segment (start 133.250828 135.870456) (end 133.250828 135.870458) (width 0.15) (layer "B.Cu") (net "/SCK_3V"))
 (segment (start 130.576726 137.895274) (end 134.05444 137.895274) (width 0.15) (layer "F.Cu") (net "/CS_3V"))
 (segment (start 134.05444 137.895274) (end 134.665042 137.284672) (width 0.15) (layer "F.Cu") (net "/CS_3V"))
 (via (at 134.665042 137.284672) (size 0.5) (drill 0.3) (layers "F.Cu" "B.Cu") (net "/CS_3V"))
 (segment (start 144.649997 133.861003) (end 145.637 132.874) (width 0.15) (layer "B.Cu") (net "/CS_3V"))
 (segment (start 134.665042 137.284672) (end 134.665042 137.006996) (width 0.15) (layer "B.Cu") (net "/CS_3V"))
 (segment (start 134.665042 137.006996) (end 137.811035 133.861003) (width 0.15) (layer "B.Cu") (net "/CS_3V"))
 (segment (start 137.811035 133.861003) (end 144.649997 133.861003) (width 0.15) (layer "B.Cu") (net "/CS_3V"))
 (segment (start 145.637 132.874) (end 145.637 129.286) (width 0.15) (layer "B.Cu") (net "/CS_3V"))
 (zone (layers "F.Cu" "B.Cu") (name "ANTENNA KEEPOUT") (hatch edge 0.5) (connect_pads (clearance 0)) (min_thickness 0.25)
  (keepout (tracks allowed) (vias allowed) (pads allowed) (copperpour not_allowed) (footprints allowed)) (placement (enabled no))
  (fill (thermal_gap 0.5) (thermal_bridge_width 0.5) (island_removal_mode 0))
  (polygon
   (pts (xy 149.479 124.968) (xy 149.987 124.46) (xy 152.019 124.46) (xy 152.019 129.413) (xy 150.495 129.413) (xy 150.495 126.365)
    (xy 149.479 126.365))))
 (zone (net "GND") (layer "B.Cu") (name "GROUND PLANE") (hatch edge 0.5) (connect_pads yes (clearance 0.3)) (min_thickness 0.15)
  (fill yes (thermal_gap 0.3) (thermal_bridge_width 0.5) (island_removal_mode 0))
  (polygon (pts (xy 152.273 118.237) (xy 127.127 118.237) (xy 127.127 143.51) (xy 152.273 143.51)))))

